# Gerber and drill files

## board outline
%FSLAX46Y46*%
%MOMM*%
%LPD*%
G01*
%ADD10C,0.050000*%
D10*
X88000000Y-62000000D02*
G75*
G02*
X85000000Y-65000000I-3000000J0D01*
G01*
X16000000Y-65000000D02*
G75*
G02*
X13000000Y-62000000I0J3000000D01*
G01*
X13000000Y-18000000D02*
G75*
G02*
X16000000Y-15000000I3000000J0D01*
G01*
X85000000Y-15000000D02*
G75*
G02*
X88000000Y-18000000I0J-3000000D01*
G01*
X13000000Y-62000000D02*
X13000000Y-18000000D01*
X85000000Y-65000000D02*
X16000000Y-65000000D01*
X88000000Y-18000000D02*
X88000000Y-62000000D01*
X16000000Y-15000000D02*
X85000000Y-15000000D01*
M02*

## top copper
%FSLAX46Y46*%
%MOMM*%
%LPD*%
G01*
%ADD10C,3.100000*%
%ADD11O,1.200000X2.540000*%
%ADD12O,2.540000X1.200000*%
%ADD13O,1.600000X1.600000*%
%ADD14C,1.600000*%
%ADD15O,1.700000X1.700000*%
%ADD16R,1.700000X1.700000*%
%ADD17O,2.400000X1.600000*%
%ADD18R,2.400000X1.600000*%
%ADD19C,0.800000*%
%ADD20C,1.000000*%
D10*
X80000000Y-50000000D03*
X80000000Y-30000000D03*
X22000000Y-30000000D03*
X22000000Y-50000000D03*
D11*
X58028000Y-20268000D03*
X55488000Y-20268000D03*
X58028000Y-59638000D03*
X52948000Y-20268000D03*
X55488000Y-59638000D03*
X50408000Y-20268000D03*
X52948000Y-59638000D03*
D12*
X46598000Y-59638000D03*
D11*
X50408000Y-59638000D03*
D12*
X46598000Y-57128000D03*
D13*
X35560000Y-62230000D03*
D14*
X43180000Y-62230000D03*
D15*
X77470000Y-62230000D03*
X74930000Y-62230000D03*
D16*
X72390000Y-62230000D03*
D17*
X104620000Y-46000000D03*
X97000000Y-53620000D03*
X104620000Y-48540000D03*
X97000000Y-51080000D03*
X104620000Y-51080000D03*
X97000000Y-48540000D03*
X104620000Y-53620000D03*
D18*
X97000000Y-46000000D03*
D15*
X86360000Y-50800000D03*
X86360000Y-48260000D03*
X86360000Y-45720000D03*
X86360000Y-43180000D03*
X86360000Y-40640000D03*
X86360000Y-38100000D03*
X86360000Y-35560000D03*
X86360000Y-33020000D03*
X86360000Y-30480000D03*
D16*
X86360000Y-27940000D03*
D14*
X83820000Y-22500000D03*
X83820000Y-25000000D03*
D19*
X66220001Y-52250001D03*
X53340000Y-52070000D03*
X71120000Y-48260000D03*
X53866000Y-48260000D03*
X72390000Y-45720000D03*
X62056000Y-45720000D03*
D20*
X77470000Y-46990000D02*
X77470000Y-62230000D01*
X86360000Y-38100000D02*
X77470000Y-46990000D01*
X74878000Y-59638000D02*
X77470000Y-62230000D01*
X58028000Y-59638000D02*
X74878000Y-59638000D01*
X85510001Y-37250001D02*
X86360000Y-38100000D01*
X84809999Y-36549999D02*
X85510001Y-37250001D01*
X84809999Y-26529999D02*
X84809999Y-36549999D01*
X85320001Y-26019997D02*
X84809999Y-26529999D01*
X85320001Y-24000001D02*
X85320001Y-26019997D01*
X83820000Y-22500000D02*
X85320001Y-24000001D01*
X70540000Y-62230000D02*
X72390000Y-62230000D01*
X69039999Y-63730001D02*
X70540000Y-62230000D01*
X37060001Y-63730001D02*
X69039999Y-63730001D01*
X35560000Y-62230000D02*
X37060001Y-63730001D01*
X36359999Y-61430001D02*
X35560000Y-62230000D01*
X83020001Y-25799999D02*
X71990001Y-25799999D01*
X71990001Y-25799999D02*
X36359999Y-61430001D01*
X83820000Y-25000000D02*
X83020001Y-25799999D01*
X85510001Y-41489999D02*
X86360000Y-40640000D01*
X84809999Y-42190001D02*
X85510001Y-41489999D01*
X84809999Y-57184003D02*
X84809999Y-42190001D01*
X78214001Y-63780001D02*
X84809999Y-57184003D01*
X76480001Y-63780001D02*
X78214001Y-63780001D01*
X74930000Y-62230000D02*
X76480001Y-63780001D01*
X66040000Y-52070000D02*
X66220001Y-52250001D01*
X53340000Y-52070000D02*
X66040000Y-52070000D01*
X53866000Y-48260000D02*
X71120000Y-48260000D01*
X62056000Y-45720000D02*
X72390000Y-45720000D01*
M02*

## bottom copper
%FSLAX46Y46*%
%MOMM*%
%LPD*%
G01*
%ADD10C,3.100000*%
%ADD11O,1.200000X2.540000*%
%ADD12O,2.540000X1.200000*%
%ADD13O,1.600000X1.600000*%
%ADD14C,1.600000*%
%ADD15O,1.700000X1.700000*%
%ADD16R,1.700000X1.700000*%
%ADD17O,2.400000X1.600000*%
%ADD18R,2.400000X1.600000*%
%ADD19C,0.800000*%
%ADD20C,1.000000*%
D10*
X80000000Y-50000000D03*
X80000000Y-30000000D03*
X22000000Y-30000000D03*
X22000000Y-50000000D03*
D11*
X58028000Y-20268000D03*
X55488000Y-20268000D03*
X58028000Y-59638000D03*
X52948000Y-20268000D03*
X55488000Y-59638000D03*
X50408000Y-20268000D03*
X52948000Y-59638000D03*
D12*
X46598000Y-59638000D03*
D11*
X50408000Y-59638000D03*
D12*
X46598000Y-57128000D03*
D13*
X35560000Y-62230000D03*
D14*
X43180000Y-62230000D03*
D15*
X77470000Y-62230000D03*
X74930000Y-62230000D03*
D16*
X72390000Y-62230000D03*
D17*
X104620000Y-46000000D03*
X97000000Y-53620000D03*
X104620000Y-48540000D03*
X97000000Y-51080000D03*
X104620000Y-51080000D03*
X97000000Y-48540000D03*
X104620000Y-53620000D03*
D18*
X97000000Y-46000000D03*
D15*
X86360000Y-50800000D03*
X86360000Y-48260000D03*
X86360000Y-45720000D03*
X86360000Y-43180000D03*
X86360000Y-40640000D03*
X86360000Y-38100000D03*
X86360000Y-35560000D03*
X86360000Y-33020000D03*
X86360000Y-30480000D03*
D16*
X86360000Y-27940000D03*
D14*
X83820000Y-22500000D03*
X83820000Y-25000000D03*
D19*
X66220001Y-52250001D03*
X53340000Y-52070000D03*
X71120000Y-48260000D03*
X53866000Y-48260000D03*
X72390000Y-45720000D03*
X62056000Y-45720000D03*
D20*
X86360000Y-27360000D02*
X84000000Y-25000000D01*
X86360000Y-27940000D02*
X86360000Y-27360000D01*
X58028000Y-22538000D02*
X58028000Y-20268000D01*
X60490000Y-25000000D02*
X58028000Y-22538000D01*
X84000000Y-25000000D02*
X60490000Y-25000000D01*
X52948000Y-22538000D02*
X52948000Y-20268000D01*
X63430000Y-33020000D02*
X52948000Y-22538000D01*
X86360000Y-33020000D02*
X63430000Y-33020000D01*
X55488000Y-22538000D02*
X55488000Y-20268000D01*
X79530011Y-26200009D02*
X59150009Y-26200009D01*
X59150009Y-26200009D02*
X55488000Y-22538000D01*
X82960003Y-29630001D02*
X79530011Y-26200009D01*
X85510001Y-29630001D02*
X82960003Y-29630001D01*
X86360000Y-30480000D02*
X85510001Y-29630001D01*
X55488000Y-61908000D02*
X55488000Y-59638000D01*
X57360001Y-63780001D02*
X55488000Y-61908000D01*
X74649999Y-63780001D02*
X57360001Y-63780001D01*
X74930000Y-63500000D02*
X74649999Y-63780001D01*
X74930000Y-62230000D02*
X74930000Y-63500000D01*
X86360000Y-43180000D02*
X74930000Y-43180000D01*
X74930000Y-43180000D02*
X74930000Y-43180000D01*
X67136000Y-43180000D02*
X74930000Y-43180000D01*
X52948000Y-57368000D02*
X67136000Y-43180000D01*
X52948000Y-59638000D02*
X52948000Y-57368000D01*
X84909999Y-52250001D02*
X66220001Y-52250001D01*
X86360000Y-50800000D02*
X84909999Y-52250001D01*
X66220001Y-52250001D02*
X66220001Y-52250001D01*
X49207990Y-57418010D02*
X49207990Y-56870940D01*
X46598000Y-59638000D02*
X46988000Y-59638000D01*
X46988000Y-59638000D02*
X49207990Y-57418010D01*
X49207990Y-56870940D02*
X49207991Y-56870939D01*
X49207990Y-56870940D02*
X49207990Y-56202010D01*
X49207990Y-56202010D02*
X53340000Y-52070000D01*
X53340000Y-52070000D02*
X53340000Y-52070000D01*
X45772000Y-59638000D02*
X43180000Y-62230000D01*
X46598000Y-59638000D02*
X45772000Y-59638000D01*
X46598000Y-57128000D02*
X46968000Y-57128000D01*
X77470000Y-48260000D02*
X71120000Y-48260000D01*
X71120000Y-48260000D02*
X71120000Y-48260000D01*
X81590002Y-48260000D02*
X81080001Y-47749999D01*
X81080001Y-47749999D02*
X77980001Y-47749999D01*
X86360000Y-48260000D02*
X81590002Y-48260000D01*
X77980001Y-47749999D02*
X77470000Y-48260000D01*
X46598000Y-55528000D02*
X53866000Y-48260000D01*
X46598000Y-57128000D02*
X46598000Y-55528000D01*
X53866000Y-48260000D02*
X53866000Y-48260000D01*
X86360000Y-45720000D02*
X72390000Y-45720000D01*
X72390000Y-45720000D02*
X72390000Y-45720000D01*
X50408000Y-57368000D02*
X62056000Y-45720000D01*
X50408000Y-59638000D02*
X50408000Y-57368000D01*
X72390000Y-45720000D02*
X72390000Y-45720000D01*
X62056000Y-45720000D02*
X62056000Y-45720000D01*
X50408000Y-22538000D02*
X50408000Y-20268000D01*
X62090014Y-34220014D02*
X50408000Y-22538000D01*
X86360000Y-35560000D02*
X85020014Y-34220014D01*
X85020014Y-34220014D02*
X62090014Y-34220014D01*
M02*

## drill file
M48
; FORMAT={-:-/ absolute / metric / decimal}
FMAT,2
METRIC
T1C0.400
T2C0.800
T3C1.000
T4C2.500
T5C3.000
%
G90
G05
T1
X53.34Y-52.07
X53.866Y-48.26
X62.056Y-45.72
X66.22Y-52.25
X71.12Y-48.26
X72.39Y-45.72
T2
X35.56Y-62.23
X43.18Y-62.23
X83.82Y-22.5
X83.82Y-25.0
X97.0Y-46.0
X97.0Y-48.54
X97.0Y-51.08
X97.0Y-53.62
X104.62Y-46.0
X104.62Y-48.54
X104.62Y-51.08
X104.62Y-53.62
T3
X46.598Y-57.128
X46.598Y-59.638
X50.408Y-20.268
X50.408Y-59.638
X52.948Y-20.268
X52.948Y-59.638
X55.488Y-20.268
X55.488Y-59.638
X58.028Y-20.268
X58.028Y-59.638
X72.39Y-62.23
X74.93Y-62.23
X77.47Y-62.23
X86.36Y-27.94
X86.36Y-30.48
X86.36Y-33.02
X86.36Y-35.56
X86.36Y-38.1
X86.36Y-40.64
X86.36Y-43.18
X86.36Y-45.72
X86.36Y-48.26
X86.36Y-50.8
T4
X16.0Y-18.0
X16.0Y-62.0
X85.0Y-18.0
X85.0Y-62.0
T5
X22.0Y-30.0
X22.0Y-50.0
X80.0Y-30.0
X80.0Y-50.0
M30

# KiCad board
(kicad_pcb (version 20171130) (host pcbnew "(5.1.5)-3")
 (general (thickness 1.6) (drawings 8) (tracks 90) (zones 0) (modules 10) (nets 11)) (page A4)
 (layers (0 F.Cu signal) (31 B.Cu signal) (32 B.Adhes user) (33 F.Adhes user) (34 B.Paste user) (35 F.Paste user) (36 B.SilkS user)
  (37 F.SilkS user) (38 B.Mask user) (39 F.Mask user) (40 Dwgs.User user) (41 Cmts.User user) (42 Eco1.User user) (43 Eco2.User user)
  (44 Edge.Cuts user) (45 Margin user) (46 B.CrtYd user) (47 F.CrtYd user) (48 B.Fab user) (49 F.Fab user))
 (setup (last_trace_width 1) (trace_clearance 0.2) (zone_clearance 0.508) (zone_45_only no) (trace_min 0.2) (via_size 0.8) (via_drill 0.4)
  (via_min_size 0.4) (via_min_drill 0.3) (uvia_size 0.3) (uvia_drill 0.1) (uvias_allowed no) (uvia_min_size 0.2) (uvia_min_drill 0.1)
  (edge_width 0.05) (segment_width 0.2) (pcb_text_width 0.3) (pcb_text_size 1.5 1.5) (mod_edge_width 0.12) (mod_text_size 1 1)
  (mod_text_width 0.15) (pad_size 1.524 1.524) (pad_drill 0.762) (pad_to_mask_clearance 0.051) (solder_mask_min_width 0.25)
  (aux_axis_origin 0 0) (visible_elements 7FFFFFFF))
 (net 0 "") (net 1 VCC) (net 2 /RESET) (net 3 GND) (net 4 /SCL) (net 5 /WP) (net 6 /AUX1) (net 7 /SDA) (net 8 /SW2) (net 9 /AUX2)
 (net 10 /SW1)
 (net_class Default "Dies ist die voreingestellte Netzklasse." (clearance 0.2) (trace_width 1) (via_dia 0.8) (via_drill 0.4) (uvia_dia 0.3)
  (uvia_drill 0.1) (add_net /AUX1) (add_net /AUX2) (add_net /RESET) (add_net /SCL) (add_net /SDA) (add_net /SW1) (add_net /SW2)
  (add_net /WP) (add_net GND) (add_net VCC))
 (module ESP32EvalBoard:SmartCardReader (layer F.Cu) (at 20 60)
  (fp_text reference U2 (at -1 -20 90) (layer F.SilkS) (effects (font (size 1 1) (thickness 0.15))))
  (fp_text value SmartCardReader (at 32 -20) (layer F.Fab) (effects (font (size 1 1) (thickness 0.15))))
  (pad "" np_thru_hole circle (at 60 -10) (size 3.1 3.1) (drill 3) (layers *.Cu *.Mask))
  (pad "" np_thru_hole circle (at 60 -30) (size 3.1 3.1) (drill 3) (layers *.Cu *.Mask))
  (pad "" np_thru_hole circle (at 2 -30) (size 3.1 3.1) (drill 3) (layers *.Cu *.Mask))
  (pad "" np_thru_hole circle (at 2 -10) (size 3.1 3.1) (drill 3) (layers *.Cu *.Mask))
  (pad 1 thru_hole oval (at 38.028 -39.732) (size 1.2 2.54) (drill 1) (layers *.Cu *.Mask) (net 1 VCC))
  (pad 2 thru_hole oval (at 35.488 -39.732) (size 1.2 2.54) (drill 1) (layers *.Cu *.Mask) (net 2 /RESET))
  (pad 5 thru_hole oval (at 38.028 -0.362) (size 1.2 2.54) (drill 1) (layers *.Cu *.Mask) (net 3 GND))
  (pad 3 thru_hole oval (at 32.948 -39.732) (size 1.2 2.54) (drill 1) (layers *.Cu *.Mask) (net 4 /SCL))
  (pad 6 thru_hole oval (at 35.488 -0.362) (size 1.2 2.54) (drill 1) (layers *.Cu *.Mask) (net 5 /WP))
  (pad 4 thru_hole oval (at 30.408 -39.732) (size 1.2 2.54) (drill 1) (layers *.Cu *.Mask) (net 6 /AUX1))
  (pad 7 thru_hole oval (at 32.948 -0.362) (size 1.2 2.54) (drill 1) (layers *.Cu *.Mask) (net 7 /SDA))
  (pad 10 thru_hole oval (at 26.598 -0.362 90) (size 1.2 2.54) (drill 1) (layers *.Cu *.Mask) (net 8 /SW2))
  (pad 8 thru_hole oval (at 30.408 -0.362) (size 1.2 2.54) (drill 1) (layers *.Cu *.Mask) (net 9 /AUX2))
  (pad 9 thru_hole oval (at 26.598 -2.872 90) (size 1.2 2.54) (drill 1) (layers *.Cu *.Mask) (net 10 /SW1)))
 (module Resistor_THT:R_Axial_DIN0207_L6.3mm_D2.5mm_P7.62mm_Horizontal (layer F.Cu) (at 43.18 62.23 180)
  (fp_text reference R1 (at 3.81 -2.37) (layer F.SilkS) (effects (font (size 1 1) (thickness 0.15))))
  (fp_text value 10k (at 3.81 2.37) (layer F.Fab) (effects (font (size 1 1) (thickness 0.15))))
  (pad 2 thru_hole oval (at 7.62 0 180) (size 1.6 1.6) (drill 0.8) (layers *.Cu *.Mask) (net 1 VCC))
  (pad 1 thru_hole circle (at 0 0 180) (size 1.6 1.6) (drill 0.8) (layers *.Cu *.Mask) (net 8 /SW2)))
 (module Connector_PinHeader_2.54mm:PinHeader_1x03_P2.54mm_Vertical (layer F.Cu) (at 72.39 62.23 90)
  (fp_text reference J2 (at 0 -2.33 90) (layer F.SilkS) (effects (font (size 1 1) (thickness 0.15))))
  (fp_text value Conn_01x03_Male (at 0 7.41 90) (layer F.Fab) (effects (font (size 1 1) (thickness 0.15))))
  (pad 3 thru_hole oval (at 0 5.08 90) (size 1.7 1.7) (drill 1) (layers *.Cu *.Mask) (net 3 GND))
  (pad 2 thru_hole oval (at 0 2.54 90) (size 1.7 1.7) (drill 1) (layers *.Cu *.Mask) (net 5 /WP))
  (pad 1 thru_hole rect (at 0 0 90) (size 1.7 1.7) (drill 1) (layers *.Cu *.Mask) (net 1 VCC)))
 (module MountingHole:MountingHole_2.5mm (layer F.Cu) (at 16 18)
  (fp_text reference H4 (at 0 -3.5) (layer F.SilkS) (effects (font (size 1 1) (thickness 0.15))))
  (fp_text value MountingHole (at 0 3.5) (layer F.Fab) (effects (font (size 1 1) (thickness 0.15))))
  (pad 1 np_thru_hole circle (at 0 0) (size 2.5 2.5) (drill 2.5) (layers *.Cu *.Mask)))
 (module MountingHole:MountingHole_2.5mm (layer F.Cu) (at 85 18)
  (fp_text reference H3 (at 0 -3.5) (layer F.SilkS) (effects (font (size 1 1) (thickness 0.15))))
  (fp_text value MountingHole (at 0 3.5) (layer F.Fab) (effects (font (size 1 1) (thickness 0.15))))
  (pad 1 np_thru_hole circle (at 0 0) (size 2.5 2.5) (drill 2.5) (layers *.Cu *.Mask)))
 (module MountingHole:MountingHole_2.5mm (layer F.Cu) (at 85 62)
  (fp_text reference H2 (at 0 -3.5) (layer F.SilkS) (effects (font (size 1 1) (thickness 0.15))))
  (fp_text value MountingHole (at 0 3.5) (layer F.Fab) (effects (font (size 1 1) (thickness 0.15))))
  (pad 1 np_thru_hole circle (at 0 0) (size 2.5 2.5) (drill 2.5) (layers *.Cu *.Mask)))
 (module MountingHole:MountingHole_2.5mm (layer F.Cu) (at 16 62)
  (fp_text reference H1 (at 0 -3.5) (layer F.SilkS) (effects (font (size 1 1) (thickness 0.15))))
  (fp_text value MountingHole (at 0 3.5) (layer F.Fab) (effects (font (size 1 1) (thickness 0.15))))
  (pad 1 np_thru_hole circle (at 0 0) (size 2.5 2.5) (drill 2.5) (layers *.Cu *.Mask)))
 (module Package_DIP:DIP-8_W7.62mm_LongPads (layer F.Cu) (at 97 46)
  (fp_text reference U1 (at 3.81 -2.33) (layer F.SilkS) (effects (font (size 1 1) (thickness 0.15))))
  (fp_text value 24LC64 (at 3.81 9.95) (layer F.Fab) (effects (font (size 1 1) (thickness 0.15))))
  (pad 8 thru_hole oval (at 7.62 0) (size 2.4 1.6) (drill 0.8) (layers *.Cu *.Mask) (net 1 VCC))
  (pad 4 thru_hole oval (at 0 7.62) (size 2.4 1.6) (drill 0.8) (layers *.Cu *.Mask) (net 3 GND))
  (pad 7 thru_hole oval (at 7.62 2.54) (size 2.4 1.6) (drill 0.8) (layers *.Cu *.Mask) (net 5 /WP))
  (pad 3 thru_hole oval (at 0 5.08) (size 2.4 1.6) (drill 0.8) (layers *.Cu *.Mask))
  (pad 6 thru_hole oval (at 7.62 5.08) (size 2.4 1.6) (drill 0.8) (layers *.Cu *.Mask) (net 4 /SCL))
  (pad 2 thru_hole oval (at 0 2.54) (size 2.4 1.6) (drill 0.8) (layers *.Cu *.Mask))
  (pad 5 thru_hole oval (at 7.62 7.62) (size 2.4 1.6) (drill 0.8) (layers *.Cu *.Mask) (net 7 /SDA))
  (pad 1 thru_hole rect (at 0 0) (size 2.4 1.6) (drill 0.8) (layers *.Cu *.Mask)))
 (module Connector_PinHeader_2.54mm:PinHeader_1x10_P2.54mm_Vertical (layer F.Cu) (at 86.36 27.94)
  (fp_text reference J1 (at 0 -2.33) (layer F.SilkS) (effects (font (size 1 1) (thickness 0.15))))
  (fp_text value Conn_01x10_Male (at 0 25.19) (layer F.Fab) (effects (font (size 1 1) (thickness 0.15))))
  (pad 10 thru_hole oval (at 0 22.86) (size 1.7 1.7) (drill 1) (layers *.Cu *.Mask) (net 8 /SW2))
  (pad 9 thru_hole oval (at 0 20.32) (size 1.7 1.7) (drill 1) (layers *.Cu *.Mask) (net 10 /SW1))
  (pad 8 thru_hole oval (at 0 17.78) (size 1.7 1.7) (drill 1) (layers *.Cu *.Mask) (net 9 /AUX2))
  (pad 7 thru_hole oval (at 0 15.24) (size 1.7 1.7) (drill 1) (layers *.Cu *.Mask) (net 7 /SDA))
  (pad 6 thru_hole oval (at 0 12.7) (size 1.7 1.7) (drill 1) (layers *.Cu *.Mask) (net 5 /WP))
  (pad 5 thru_hole oval (at 0 10.16) (size 1.7 1.7) (drill 1) (layers *.Cu *.Mask) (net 3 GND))
  (pad 4 thru_hole oval (at 0 7.62) (size 1.7 1.7) (drill 1) (layers *.Cu *.Mask) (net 6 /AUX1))
  (pad 3 thru_hole oval (at 0 5.08) (size 1.7 1.7) (drill 1) (layers *.Cu *.Mask) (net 4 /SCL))
  (pad 2 thru_hole oval (at 0 2.54) (size 1.7 1.7) (drill 1) (layers *.Cu *.Mask) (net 2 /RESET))
  (pad 1 thru_hole rect (at 0 0) (size 1.7 1.7) (drill 1) (layers *.Cu *.Mask) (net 1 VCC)))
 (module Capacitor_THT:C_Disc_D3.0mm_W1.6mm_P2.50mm (layer F.Cu) (at 83.82 25 90)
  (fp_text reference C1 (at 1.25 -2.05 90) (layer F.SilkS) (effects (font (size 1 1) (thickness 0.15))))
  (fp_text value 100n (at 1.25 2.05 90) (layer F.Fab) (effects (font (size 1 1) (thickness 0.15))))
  (pad 2 thru_hole circle (at 2.5 0 90) (size 1.6 1.6) (drill 0.8) (layers *.Cu *.Mask) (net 3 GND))
  (pad 1 thru_hole circle (at 0 0 90) (size 1.6 1.6) (drill 0.8) (layers *.Cu *.Mask) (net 1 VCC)))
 (gr_arc (start 85 62) (end 85 65) (angle -90) (layer Edge.Cuts) (width 0.05))
 (gr_arc (start 16 62) (end 13 62) (angle -90) (layer Edge.Cuts) (width 0.05))
 (gr_arc (start 16 18) (end 16 15) (angle -90) (layer Edge.Cuts) (width 0.05))
 (gr_arc (start 85 18) (end 88 18) (angle -90) (layer Edge.Cuts) (width 0.05))
 (gr_line (start 13 62) (end 13 18) (layer Edge.Cuts) (width 0.05))
 (gr_line (start 85 65) (end 16 65) (layer Edge.Cuts) (width 0.05))
 (gr_line (start 88 18) (end 88 62) (layer Edge.Cuts) (width 0.05))
 (gr_line (start 16 15) (end 85 15) (layer Edge.Cuts) (width 0.05))
 (segment (start 77.47 46.99) (end 77.47 62.23) (width 1) (layer F.Cu) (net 3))
 (segment (start 86.36 38.1) (end 77.47 46.99) (width 1) (layer F.Cu) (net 3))
 (segment (start 74.878 59.638) (end 77.47 62.23) (width 1) (layer F.Cu) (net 3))
 (segment (start 58.028 59.638) (end 74.878 59.638) (width 1) (layer F.Cu) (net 3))
 (segment (start 85.510001 37.250001) (end 86.36 38.1) (width 1) (layer F.Cu) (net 3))
 (segment (start 84.809999 36.549999) (end 85.510001 37.250001) (width 1) (layer F.Cu) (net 3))
 (segment (start 84.809999 26.529999) (end 84.809999 36.549999) (width 1) (layer F.Cu) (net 3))
 (segment (start 85.320001 26.019997) (end 84.809999 26.529999) (width 1) (layer F.Cu) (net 3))
 (segment (start 85.320001 24.000001) (end 85.320001 26.019997) (width 1) (layer F.Cu) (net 3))
 (segment (start 83.82 22.5) (end 85.320001 24.000001) (width 1) (layer F.Cu) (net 3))
 (segment (start 86.36 27.36) (end 84 25) (width 1) (layer B.Cu) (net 1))
 (segment (start 86.36 27.94) (end 86.36 27.36) (width 1) (layer B.Cu) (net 1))
 (segment (start 58.028 22.538) (end 58.028 20.268) (width 1) (layer B.Cu) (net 1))
 (segment (start 60.49 25) (end 58.028 22.538) (width 1) (layer B.Cu) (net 1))
 (segment (start 84 25) (end 60.49 25) (width 1) (layer B.Cu) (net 1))
 (segment (start 70.54 62.23) (end 72.39 62.23) (width 1) (layer F.Cu) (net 1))
 (segment (start 69.039999 63.730001) (end 70.54 62.23) (width 1) (layer F.Cu) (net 1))
 (segment (start 37.060001 63.730001) (end 69.039999 63.730001) (width 1) (layer F.Cu) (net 1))
 (segment (start 35.56 62.23) (end 37.060001 63.730001) (width 1) (layer F.Cu) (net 1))
 (segment (start 36.359999 61.430001) (end 35.56 62.23) (width 1) (layer F.Cu) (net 1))
 (segment (start 83.020001 25.799999) (end 71.990001 25.799999) (width 1) (layer F.Cu) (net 1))
 (segment (start 71.990001 25.799999) (end 36.359999 61.430001) (width 1) (layer F.Cu) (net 1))
 (segment (start 83.82 25) (end 83.020001 25.799999) (width 1) (layer F.Cu) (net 1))
 (segment (start 52.948 22.538) (end 52.948 20.268) (width 1) (layer B.Cu) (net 4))
 (segment (start 63.43 33.02) (end 52.948 22.538) (width 1) (layer B.Cu) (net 4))
 (segment (start 86.36 33.02) (end 63.43 33.02) (width 1) (layer B.Cu) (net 4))
 (segment (start 55.488 22.538) (end 55.488 20.268) (width 1) (layer B.Cu) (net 2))
 (segment (start 79.530011 26.200009) (end 59.150009 26.200009) (width 1) (layer B.Cu) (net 2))
 (segment (start 59.150009 26.200009) (end 55.488 22.538) (width 1) (layer B.Cu) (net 2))
 (segment (start 82.960003 29.630001) (end 79.530011 26.200009) (width 1) (layer B.Cu) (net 2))
 (segment (start 85.510001 29.630001) (end 82.960003 29.630001) (width 1) (layer B.Cu) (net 2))
 (segment (start 86.36 30.48) (end 85.510001 29.630001) (width 1) (layer B.Cu) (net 2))
 (segment (start 85.510001 41.489999) (end 86.36 40.64) (width 1) (layer F.Cu) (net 5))
 (segment (start 84.809999 42.190001) (end 85.510001 41.489999) (width 1) (layer F.Cu) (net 5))
 (segment (start 84.809999 57.184003) (end 84.809999 42.190001) (width 1) (layer F.Cu) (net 5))
 (segment (start 78.214001 63.780001) (end 84.809999 57.184003) (width 1) (layer F.Cu) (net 5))
 (segment (start 76.480001 63.780001) (end 78.214001 63.780001) (width 1) (layer F.Cu) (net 5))
 (segment (start 74.93 62.23) (end 76.480001 63.780001) (width 1) (layer F.Cu) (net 5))
 (segment (start 55.488 61.908) (end 55.488 59.638) (width 1) (layer B.Cu) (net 5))
 (segment (start 57.360001 63.780001) (end 55.488 61.908) (width 1) (layer B.Cu) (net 5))
 (segment (start 74.649999 63.780001) (end 57.360001 63.780001) (width 1) (layer B.Cu) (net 5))
 (segment (start 74.93 63.5) (end 74.649999 63.780001) (width 1) (layer B.Cu) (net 5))
 (segment (start 74.93 62.23) (end 74.93 63.5) (width 1) (layer B.Cu) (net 5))
 (segment (start 86.36 43.18) (end 74.93 43.18) (width 1) (layer B.Cu) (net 7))
 (segment (start 74.93 43.18) (end 74.93 43.18) (width 1) (layer B.Cu) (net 7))
 (segment (start 67.136 43.18) (end 74.93 43.18) (width 1) (layer B.Cu) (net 7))
 (segment (start 52.948 57.368) (end 67.136 43.18) (width 1) (layer B.Cu) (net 7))
 (segment (start 52.948 59.638) (end 52.948 57.368) (width 1) (layer B.Cu) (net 7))
 (segment (start 84.909999 52.250001) (end 66.220001 52.250001) (width 1) (layer B.Cu) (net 8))
 (segment (start 86.36 50.8) (end 84.909999 52.250001) (width 1) (layer B.Cu) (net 8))
 (segment (start 66.220001 52.250001) (end 66.220001 52.250001) (width 1) (layer B.Cu) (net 8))
 (via (at 66.220001 52.250001) (size 0.8) (drill 0.4) (layers F.Cu B.Cu) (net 8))
 (segment (start 49.20799 57.41801) (end 49.20799 56.87094) (width 1) (layer B.Cu) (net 8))
 (segment (start 46.598 59.638) (end 46.988 59.638) (width 1) (layer B.Cu) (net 8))
 (segment (start 46.988 59.638) (end 49.20799 57.41801) (width 1) (layer B.Cu) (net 8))
 (segment (start 49.20799 56.87094) (end 49.207991 56.870939) (width 1) (layer B.Cu) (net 8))
 (segment (start 49.20799 56.87094) (end 49.20799 56.20201) (width 1) (layer B.Cu) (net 8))
 (segment (start 49.20799 56.20201) (end 53.34 52.07) (width 1) (layer B.Cu) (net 8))
 (segment (start 53.34 52.07) (end 53.34 52.07) (width 1) (layer B.Cu) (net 8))
 (via (at 53.34 52.07) (size 0.8) (drill 0.4) (layers F.Cu B.Cu) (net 8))
 (segment (start 66.04 52.07) (end 66.220001 52.250001) (width 1) (layer F.Cu) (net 8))
 (segment (start 53.34 52.07) (end 66.04 52.07) (width 1) (layer F.Cu) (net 8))
 (segment (start 45.772 59.638) (end 43.18 62.23) (width 1) (layer B.Cu) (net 8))
 (segment (start 46.598 59.638) (end 45.772 59.638) (width 1) (layer B.Cu) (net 8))
 (segment (start 46.598 57.128) (end 46.968 57.128) (width 1) (layer B.Cu) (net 10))
 (segment (start 77.47 48.26) (end 71.12 48.26) (width 1) (layer B.Cu) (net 10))
 (segment (start 71.12 48.26) (end 71.12 48.26) (width 1) (layer B.Cu) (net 10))
 (segment (start 81.590002 48.26) (end 81.080001 47.749999) (width 1) (layer B.Cu) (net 10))
 (segment (start 81.080001 47.749999) (end 77.980001 47.749999) (width 1) (layer B.Cu) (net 10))
 (segment (start 86.36 48.26) (end 81.590002 48.26) (width 1) (layer B.Cu) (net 10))
 (segment (start 77.980001 47.749999) (end 77.47 48.26) (width 1) (layer B.Cu) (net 10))
 (via (at 71.12 48.26) (size 0.8) (drill 0.4) (layers F.Cu B.Cu) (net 10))
 (segment (start 46.598 55.528) (end 53.866 48.26) (width 1) (layer B.Cu) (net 10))
 (segment (start 46.598 57.128) (end 46.598 55.528) (width 1) (layer B.Cu) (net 10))
 (segment (start 53.866 48.26) (end 53.866 48.26) (width 1) (layer B.Cu) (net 10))
 (via (at 53.866 48.26) (size 0.8) (drill 0.4) (layers F.Cu B.Cu) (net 10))
 (segment (start 53.866 48.26) (end 71.12 48.26) (width 1) (layer F.Cu) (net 10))
 (segment (start 86.36 45.72) (end 72.39 45.72) (width 1) (layer B.Cu) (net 9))
 (segment (start 72.39 45.72) (end 72.39 45.72) (width 1) (layer B.Cu) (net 9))
 (segment (start 50.408 57.368) (end 62.056 45.72) (width 1) (layer B.Cu) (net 9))
 (segment (start 50.408 59.638) (end 50.408 57.368) (width 1) (layer B.Cu) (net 9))
 (segment (start 72.39 45.72) (end 72.39 45.72) (width 1) (layer B.Cu) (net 9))
 (via (at 72.39 45.72) (size 0.8) (drill 0.4) (layers F.Cu B.Cu) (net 9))
 (segment (start 62.056 45.72) (end 62.056 45.72) (width 1) (layer B.Cu) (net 9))
 (via (at 62.056 45.72) (size 0.8) (drill 0.4) (layers F.Cu B.Cu) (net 9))
 (segment (start 62.056 45.72) (end 72.39 45.72) (width 1) (layer F.Cu) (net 9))
 (segment (start 50.408 22.538) (end 50.408 20.268) (width 1) (layer B.Cu) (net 6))
 (segment (start 62.090014 34.220014) (end 50.408 22.538) (width 1) (layer B.Cu) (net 6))
 (segment (start 86.36 35.56) (end 85.020014 34.220014) (width 1) (layer B.Cu) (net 6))
 (segment (start 85.020014 34.220014) (end 62.090014 34.220014) (width 1) (layer B.Cu) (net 6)))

